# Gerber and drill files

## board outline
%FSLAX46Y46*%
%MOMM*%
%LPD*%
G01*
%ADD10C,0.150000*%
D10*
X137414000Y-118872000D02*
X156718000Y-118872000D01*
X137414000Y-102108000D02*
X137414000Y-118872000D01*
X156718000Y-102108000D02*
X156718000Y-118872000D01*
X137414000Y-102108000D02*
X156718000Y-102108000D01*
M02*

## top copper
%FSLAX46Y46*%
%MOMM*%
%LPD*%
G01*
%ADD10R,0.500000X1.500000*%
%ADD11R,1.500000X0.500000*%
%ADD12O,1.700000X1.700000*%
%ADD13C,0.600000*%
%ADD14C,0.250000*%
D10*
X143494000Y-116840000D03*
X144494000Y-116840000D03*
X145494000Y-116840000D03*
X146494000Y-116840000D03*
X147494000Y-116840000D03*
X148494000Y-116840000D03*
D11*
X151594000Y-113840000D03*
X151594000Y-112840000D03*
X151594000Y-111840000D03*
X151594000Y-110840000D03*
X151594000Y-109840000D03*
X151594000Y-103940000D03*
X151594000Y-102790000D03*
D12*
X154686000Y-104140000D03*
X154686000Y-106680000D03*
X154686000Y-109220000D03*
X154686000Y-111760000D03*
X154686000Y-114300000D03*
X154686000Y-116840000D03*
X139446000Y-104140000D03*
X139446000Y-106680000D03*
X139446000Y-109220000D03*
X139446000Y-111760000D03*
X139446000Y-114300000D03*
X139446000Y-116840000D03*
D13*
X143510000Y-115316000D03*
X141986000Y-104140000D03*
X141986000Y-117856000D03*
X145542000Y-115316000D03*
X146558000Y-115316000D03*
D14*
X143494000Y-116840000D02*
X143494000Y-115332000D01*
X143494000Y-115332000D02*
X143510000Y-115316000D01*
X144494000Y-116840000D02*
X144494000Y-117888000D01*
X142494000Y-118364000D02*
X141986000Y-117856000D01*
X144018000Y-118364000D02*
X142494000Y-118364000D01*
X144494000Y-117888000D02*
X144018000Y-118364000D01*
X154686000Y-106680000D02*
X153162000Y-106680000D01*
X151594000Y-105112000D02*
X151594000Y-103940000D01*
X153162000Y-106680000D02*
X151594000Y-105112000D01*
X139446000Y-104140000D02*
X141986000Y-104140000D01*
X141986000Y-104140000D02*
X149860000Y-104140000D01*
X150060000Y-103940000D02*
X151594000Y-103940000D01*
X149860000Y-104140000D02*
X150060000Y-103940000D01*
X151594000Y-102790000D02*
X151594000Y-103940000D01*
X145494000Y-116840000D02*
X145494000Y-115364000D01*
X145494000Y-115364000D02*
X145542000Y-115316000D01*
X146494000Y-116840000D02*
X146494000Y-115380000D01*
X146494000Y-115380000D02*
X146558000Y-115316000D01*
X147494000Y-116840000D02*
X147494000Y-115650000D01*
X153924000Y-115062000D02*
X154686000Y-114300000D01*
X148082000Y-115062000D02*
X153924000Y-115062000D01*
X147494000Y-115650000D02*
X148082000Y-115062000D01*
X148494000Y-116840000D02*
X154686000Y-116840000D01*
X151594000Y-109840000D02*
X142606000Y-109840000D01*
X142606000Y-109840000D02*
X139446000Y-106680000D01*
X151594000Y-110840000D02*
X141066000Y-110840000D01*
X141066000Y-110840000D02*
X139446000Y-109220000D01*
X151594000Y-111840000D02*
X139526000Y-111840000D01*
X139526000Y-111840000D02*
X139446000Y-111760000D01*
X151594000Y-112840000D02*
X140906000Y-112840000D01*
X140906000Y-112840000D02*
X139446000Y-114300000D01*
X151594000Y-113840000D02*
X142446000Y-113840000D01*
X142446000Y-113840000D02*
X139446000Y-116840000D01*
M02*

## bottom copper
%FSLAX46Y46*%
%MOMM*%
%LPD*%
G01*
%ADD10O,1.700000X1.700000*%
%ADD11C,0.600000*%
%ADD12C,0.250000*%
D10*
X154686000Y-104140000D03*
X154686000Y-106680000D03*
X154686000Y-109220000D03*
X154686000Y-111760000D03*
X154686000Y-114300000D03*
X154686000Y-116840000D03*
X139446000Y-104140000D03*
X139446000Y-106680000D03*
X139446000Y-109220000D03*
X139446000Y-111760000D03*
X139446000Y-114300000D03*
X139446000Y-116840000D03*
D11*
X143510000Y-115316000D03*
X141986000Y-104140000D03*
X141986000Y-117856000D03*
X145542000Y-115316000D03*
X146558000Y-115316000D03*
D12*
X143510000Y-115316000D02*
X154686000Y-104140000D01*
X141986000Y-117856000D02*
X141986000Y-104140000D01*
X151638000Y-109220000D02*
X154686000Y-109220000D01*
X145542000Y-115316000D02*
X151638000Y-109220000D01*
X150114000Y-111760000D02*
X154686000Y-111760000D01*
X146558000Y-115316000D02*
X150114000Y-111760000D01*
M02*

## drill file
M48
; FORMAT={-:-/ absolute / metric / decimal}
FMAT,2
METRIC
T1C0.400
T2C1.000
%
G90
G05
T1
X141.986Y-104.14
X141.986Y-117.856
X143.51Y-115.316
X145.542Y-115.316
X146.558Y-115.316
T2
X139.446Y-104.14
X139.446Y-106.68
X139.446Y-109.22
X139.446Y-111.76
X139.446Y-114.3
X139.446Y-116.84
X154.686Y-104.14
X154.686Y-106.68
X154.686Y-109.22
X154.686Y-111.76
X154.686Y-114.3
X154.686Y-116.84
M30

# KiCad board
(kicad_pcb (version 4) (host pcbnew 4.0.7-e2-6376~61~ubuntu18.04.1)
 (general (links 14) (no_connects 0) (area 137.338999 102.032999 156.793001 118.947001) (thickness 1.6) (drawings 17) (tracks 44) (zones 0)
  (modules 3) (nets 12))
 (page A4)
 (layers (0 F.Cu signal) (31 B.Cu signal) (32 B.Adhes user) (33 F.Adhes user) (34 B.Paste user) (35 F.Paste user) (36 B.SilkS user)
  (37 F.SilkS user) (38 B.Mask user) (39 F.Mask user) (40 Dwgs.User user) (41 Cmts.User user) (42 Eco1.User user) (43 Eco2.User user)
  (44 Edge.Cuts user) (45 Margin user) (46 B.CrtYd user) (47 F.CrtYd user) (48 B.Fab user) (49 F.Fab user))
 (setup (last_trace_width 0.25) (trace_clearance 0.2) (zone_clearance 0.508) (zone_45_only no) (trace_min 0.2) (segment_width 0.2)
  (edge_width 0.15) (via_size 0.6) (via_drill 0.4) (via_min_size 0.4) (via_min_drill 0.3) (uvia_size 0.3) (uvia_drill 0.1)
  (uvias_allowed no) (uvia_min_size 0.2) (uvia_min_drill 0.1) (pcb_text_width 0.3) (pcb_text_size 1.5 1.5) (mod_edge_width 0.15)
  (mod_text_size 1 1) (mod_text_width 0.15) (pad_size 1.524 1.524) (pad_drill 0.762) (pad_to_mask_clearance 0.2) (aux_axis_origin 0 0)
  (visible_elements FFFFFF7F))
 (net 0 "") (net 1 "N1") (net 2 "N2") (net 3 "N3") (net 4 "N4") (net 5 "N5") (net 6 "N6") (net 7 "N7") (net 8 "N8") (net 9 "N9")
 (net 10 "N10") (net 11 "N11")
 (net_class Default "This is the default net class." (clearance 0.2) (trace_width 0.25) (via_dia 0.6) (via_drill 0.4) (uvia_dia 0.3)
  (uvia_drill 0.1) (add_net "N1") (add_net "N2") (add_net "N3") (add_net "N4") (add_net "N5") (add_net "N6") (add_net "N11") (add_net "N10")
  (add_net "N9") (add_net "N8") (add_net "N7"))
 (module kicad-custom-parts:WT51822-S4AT (layer F.Cu) (at 142.494 116.84 90)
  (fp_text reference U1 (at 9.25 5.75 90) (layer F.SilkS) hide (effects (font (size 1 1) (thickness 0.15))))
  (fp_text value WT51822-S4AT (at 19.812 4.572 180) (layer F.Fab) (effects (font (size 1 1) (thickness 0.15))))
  (pad 1 smd rect (at 0 1 90) (size 1.5 0.5) (layers F.Cu F.Paste F.Mask) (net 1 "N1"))
  (pad 2 smd rect (at 0 2 90) (size 1.5 0.5) (layers F.Cu F.Paste F.Mask) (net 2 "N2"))
  (pad 3 smd rect (at 0 3 90) (size 1.5 0.5) (layers F.Cu F.Paste F.Mask) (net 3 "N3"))
  (pad 4 smd rect (at 0 4 90) (size 1.5 0.5) (layers F.Cu F.Paste F.Mask) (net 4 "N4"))
  (pad 5 smd rect (at 0 5 90) (size 1.5 0.5) (layers F.Cu F.Paste F.Mask) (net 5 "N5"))
  (pad 6 smd rect (at 0 6 90) (size 1.5 0.5) (layers F.Cu F.Paste F.Mask) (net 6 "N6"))
  (pad 7 smd rect (at 3 9.1 90) (size 0.5 1.5) (layers F.Cu F.Paste F.Mask) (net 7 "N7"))
  (pad 8 smd rect (at 4 9.1 90) (size 0.5 1.5) (layers F.Cu F.Paste F.Mask) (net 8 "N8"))
  (pad 9 smd rect (at 5 9.1 90) (size 0.5 1.5) (layers F.Cu F.Paste F.Mask) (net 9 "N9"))
  (pad 10 smd rect (at 6 9.1 90) (size 0.5 1.5) (layers F.Cu F.Paste F.Mask) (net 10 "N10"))
  (pad 11 smd rect (at 7 9.1 90) (size 0.5 1.5) (layers F.Cu F.Paste F.Mask) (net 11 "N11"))
  (pad 12 smd rect (at 12.9 9.1 90) (size 0.5 1.5) (layers F.Cu F.Paste F.Mask) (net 2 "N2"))
  (pad 13 smd rect (at 14.05 9.1 90) (size 0.5 1.5) (layers F.Cu F.Paste F.Mask) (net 2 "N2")))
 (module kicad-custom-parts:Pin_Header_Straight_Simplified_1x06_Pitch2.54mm (layer F.Cu) (at 154.686 104.14)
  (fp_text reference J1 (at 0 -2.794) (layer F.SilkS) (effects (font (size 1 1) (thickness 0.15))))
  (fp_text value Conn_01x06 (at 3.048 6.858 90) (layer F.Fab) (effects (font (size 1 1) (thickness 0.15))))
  (pad 1 thru_hole oval (at 0 0) (size 1.7 1.7) (drill 1) (layers *.Cu *.Mask) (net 1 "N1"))
  (pad 2 thru_hole oval (at 0 2.54) (size 1.7 1.7) (drill 1) (layers *.Cu *.Mask) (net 2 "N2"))
  (pad 3 thru_hole oval (at 0 5.08) (size 1.7 1.7) (drill 1) (layers *.Cu *.Mask) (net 3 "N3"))
  (pad 4 thru_hole oval (at 0 7.62) (size 1.7 1.7) (drill 1) (layers *.Cu *.Mask) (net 4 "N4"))
  (pad 5 thru_hole oval (at 0 10.16) (size 1.7 1.7) (drill 1) (layers *.Cu *.Mask) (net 5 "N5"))
  (pad 6 thru_hole oval (at 0 12.7) (size 1.7 1.7) (drill 1) (layers *.Cu *.Mask) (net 6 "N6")))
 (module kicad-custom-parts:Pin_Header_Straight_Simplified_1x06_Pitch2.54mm (layer F.Cu) (at 139.446 104.14)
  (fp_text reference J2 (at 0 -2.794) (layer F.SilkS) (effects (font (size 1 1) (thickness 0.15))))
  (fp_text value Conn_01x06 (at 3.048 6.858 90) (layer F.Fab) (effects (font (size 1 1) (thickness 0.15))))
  (pad 1 thru_hole oval (at 0 0) (size 1.7 1.7) (drill 1) (layers *.Cu *.Mask) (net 2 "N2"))
  (pad 2 thru_hole oval (at 0 2.54) (size 1.7 1.7) (drill 1) (layers *.Cu *.Mask) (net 11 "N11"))
  (pad 3 thru_hole oval (at 0 5.08) (size 1.7 1.7) (drill 1) (layers *.Cu *.Mask) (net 10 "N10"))
  (pad 4 thru_hole oval (at 0 7.62) (size 1.7 1.7) (drill 1) (layers *.Cu *.Mask) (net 9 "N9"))
  (pad 5 thru_hole oval (at 0 10.16) (size 1.7 1.7) (drill 1) (layers *.Cu *.Mask) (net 8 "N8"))
  (pad 6 thru_hole oval (at 0 12.7) (size 1.7 1.7) (drill 1) (layers *.Cu *.Mask) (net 7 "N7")))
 (gr_line (start 137.414 118.872) (end 156.718 118.872) (angle 90) (layer Edge.Cuts) (width 0.15))
 (gr_line (start 137.414 102.108) (end 137.414 118.872) (angle 90) (layer Edge.Cuts) (width 0.15))
 (gr_line (start 156.718 102.108) (end 156.718 118.872) (angle 90) (layer Edge.Cuts) (width 0.15))
 (gr_line (start 137.414 102.108) (end 156.718 102.108) (angle 90) (layer Edge.Cuts) (width 0.15))
 (segment (start 143.494 116.84) (end 143.494 115.332) (width 0.25) (layer F.Cu) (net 1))
 (segment (start 143.51 115.316) (end 154.686 104.14) (width 0.25) (layer B.Cu) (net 1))
 (via (at 143.51 115.316) (size 0.6) (drill 0.4) (layers F.Cu B.Cu) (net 1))
 (segment (start 143.494 115.332) (end 143.51 115.316) (width 0.25) (layer F.Cu) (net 1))
 (segment (start 144.494 116.84) (end 144.494 117.888) (width 0.25) (layer F.Cu) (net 2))
 (via (at 141.986 104.14) (size 0.6) (drill 0.4) (layers F.Cu B.Cu) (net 2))
 (segment (start 141.986 117.856) (end 141.986 104.14) (width 0.25) (layer B.Cu) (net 2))
 (via (at 141.986 117.856) (size 0.6) (drill 0.4) (layers F.Cu B.Cu) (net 2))
 (segment (start 142.494 118.364) (end 141.986 117.856) (width 0.25) (layer F.Cu) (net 2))
 (segment (start 144.018 118.364) (end 142.494 118.364) (width 0.25) (layer F.Cu) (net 2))
 (segment (start 144.494 117.888) (end 144.018 118.364) (width 0.25) (layer F.Cu) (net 2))
 (segment (start 154.686 106.68) (end 153.162 106.68) (width 0.25) (layer F.Cu) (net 2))
 (segment (start 151.594 105.112) (end 151.594 103.94) (width 0.25) (layer F.Cu) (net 2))
 (segment (start 153.162 106.68) (end 151.594 105.112) (width 0.25) (layer F.Cu) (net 2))
 (segment (start 139.446 104.14) (end 141.986 104.14) (width 0.25) (layer F.Cu) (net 2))
 (segment (start 141.986 104.14) (end 149.86 104.14) (width 0.25) (layer F.Cu) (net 2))
 (segment (start 150.06 103.94) (end 151.594 103.94) (width 0.25) (layer F.Cu) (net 2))
 (segment (start 149.86 104.14) (end 150.06 103.94) (width 0.25) (layer F.Cu) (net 2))
 (segment (start 151.594 102.79) (end 151.594 103.94) (width 0.25) (layer F.Cu) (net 2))
 (segment (start 145.494 116.84) (end 145.494 115.364) (width 0.25) (layer F.Cu) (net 3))
 (segment (start 151.638 109.22) (end 154.686 109.22) (width 0.25) (layer B.Cu) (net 3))
 (segment (start 145.542 115.316) (end 151.638 109.22) (width 0.25) (layer B.Cu) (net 3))
 (via (at 145.542 115.316) (size 0.6) (drill 0.4) (layers F.Cu B.Cu) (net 3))
 (segment (start 145.494 115.364) (end 145.542 115.316) (width 0.25) (layer F.Cu) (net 3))
 (segment (start 146.494 116.84) (end 146.494 115.38) (width 0.25) (layer F.Cu) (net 4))
 (segment (start 150.114 111.76) (end 154.686 111.76) (width 0.25) (layer B.Cu) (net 4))
 (segment (start 146.558 115.316) (end 150.114 111.76) (width 0.25) (layer B.Cu) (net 4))
 (via (at 146.558 115.316) (size 0.6) (drill 0.4) (layers F.Cu B.Cu) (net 4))
 (segment (start 146.494 115.38) (end 146.558 115.316) (width 0.25) (layer F.Cu) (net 4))
 (segment (start 147.494 116.84) (end 147.494 115.65) (width 0.25) (layer F.Cu) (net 5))
 (segment (start 153.924 115.062) (end 154.686 114.3) (width 0.25) (layer F.Cu) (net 5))
 (segment (start 148.082 115.062) (end 153.924 115.062) (width 0.25) (layer F.Cu) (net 5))
 (segment (start 147.494 115.65) (end 148.082 115.062) (width 0.25) (layer F.Cu) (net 5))
 (segment (start 148.494 116.84) (end 154.686 116.84) (width 0.25) (layer F.Cu) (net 6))
 (segment (start 151.594 109.84) (end 142.606 109.84) (width 0.25) (layer F.Cu) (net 11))
 (segment (start 142.606 109.84) (end 139.446 106.68) (width 0.25) (layer F.Cu) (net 11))
 (segment (start 151.594 110.84) (end 141.066 110.84) (width 0.25) (layer F.Cu) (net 10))
 (segment (start 141.066 110.84) (end 139.446 109.22) (width 0.25) (layer F.Cu) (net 10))
 (segment (start 151.594 111.84) (end 139.526 111.84) (width 0.25) (layer F.Cu) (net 9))
 (segment (start 139.526 111.84) (end 139.446 111.76) (width 0.25) (layer F.Cu) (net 9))
 (segment (start 151.594 112.84) (end 140.906 112.84) (width 0.25) (layer F.Cu) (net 8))
 (segment (start 140.906 112.84) (end 139.446 114.3) (width 0.25) (layer F.Cu) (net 8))
 (segment (start 151.594 113.84) (end 142.446 113.84) (width 0.25) (layer F.Cu) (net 7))
 (segment (start 142.446 113.84) (end 139.446 116.84) (width 0.25) (layer F.Cu) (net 7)))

